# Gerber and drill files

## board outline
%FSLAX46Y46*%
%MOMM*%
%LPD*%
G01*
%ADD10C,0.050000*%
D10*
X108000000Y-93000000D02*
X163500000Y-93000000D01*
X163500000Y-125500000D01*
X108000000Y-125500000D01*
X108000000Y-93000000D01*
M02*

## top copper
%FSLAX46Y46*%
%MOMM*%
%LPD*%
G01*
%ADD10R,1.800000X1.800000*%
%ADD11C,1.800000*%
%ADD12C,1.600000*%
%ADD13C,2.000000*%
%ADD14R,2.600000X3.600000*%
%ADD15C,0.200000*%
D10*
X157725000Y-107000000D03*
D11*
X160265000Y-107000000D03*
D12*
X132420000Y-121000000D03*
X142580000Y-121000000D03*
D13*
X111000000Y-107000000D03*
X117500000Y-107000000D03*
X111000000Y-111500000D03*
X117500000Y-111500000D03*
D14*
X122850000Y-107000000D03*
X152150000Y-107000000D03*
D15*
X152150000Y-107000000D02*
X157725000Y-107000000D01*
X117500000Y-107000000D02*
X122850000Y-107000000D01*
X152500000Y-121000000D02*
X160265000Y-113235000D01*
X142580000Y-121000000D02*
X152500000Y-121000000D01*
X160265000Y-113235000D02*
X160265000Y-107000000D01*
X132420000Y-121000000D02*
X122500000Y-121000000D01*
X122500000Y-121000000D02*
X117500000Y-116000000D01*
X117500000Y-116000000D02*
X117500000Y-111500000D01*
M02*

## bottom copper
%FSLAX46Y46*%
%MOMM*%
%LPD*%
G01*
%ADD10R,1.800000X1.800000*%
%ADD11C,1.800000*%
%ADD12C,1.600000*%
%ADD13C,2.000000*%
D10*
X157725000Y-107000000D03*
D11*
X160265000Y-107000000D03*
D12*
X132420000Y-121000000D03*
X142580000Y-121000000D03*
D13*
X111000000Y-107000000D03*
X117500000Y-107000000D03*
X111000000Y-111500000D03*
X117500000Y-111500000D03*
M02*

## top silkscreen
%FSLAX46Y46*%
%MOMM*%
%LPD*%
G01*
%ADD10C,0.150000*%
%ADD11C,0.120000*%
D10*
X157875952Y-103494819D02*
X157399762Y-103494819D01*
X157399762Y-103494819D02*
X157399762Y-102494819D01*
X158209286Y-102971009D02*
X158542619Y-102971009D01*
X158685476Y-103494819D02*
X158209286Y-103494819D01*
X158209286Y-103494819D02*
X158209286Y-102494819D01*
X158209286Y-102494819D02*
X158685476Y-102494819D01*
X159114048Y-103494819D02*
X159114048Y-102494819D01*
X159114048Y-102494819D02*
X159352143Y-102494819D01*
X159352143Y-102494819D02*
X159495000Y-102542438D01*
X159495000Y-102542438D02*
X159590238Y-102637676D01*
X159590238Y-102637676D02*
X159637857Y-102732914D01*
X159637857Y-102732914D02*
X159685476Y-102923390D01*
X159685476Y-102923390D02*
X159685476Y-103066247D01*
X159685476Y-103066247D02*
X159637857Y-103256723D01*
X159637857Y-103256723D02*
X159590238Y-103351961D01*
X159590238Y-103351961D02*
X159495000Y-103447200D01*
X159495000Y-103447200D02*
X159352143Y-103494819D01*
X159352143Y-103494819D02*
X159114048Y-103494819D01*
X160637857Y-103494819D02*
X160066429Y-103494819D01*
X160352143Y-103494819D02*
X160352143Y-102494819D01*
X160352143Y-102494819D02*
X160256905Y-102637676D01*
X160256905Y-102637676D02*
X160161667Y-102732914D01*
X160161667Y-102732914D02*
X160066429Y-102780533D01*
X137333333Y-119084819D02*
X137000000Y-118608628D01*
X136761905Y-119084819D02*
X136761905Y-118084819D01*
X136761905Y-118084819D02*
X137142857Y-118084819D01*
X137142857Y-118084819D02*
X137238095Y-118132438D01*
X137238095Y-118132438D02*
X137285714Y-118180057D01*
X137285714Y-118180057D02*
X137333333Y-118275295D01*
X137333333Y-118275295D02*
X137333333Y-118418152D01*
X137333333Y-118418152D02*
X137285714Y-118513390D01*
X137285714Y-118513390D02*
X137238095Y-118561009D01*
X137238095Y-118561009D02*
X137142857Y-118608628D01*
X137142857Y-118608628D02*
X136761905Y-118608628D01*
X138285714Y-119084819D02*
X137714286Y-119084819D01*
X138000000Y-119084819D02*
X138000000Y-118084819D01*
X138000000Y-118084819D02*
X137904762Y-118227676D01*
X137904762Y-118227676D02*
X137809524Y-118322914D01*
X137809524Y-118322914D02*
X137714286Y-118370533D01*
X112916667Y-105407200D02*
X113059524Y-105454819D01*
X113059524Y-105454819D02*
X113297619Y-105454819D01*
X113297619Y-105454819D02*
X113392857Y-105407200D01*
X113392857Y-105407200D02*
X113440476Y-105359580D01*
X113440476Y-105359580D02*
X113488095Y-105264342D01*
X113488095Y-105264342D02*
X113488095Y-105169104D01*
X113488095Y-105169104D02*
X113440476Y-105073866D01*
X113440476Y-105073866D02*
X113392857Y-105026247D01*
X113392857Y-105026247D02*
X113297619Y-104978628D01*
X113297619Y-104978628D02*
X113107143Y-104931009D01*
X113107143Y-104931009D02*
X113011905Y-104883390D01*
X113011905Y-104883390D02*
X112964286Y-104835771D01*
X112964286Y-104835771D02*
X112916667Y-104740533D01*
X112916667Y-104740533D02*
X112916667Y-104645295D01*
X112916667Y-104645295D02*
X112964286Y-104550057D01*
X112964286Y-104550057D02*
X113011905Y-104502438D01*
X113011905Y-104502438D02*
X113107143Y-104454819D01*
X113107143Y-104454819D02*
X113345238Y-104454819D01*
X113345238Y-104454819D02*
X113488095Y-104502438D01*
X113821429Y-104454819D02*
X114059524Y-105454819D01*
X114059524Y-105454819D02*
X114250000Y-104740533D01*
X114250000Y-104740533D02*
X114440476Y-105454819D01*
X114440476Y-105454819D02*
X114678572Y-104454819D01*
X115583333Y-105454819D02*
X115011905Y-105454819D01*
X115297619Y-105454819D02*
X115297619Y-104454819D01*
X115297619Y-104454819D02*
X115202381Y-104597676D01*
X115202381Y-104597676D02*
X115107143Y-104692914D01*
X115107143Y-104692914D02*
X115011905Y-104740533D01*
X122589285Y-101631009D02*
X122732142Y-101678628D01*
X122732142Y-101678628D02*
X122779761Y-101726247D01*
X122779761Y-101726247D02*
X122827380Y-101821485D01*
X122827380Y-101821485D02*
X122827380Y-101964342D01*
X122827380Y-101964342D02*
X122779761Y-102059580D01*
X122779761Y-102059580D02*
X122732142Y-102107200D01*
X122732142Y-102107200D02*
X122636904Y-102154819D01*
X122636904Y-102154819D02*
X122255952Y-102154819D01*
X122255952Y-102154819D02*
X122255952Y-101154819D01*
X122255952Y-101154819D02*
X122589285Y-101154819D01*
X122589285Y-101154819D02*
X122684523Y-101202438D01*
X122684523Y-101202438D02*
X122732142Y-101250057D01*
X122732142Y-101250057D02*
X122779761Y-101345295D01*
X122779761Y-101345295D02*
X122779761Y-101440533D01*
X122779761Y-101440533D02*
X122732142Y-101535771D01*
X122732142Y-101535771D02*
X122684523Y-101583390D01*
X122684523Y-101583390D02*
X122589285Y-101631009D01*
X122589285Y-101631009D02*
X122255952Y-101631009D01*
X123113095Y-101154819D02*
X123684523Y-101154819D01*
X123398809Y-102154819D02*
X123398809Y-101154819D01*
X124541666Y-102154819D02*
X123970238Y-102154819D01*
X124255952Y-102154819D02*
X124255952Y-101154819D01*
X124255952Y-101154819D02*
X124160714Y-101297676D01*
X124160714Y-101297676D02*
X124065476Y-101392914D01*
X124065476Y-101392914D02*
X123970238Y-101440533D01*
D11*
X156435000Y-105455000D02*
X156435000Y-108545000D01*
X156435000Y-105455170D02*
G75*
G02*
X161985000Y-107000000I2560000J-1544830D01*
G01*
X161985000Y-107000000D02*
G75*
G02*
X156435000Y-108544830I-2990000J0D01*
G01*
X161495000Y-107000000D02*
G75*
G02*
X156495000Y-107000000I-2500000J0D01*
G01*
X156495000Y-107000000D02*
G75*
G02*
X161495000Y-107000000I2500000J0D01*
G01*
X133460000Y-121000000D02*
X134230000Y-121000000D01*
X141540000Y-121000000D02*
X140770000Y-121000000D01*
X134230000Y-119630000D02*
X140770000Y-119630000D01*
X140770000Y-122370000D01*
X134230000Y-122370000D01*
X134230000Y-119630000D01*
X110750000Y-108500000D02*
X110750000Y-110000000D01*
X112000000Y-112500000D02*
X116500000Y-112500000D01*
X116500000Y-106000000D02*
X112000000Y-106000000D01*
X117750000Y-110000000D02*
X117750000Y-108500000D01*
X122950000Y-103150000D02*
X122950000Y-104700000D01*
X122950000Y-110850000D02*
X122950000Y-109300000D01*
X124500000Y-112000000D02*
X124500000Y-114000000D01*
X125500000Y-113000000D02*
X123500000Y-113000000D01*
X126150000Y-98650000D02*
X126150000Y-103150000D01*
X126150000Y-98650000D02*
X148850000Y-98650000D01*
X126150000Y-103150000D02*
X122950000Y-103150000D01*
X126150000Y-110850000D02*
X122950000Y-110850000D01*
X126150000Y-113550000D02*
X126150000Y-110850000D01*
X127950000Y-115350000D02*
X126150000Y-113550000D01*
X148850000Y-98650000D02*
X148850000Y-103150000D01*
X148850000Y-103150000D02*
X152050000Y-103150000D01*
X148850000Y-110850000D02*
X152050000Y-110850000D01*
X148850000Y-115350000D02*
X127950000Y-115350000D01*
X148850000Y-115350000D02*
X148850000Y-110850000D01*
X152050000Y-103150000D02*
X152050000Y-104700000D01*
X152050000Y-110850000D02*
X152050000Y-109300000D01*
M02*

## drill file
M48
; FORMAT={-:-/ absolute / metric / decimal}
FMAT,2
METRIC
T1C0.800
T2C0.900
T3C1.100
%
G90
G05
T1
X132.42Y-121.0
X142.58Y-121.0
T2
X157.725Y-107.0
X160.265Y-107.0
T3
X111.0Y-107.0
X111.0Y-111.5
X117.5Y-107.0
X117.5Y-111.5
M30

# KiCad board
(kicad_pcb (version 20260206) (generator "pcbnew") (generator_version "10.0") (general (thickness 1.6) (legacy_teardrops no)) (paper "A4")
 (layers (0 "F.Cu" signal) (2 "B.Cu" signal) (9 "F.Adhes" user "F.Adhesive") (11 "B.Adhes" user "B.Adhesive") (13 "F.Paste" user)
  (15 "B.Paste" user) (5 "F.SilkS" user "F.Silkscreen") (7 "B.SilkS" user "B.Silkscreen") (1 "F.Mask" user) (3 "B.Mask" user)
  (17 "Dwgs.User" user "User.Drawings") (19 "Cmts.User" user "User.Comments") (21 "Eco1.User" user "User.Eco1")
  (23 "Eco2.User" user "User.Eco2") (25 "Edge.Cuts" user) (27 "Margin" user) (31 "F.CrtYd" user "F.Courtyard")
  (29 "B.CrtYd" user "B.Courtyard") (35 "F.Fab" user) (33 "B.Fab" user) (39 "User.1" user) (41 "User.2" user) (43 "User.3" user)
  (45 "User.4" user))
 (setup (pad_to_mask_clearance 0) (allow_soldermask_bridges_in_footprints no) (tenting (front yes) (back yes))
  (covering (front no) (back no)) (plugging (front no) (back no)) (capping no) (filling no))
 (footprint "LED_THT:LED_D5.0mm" (layer "F.Cu") (at 157.725 107)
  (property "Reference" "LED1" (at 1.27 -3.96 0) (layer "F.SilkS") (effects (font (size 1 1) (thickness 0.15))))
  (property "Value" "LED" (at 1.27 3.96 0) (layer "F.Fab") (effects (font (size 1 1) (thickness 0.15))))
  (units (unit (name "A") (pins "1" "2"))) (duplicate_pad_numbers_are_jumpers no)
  (fp_line (start -1.29 -1.545) (end -1.29 1.545) (stroke (width 0.12) (type solid)) (layer "F.SilkS"))
  (fp_arc (start -1.29 -1.54483) (mid 2.071779 -2.880495) (end 4.26 0) (stroke (width 0.12) (type solid)) (layer "F.SilkS"))
  (fp_arc (start 4.26 0) (mid 2.071779 2.880495) (end -1.29 1.54483) (stroke (width 0.12) (type solid)) (layer "F.SilkS"))
  (fp_circle (center 1.27 0) (end 3.77 0) (stroke (width 0.12) (type solid)) (fill no) (layer "F.SilkS"))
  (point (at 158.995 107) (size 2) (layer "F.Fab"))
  (pad "1" thru_hole rect (at 0 0) (size 1.8 1.8) (drill 0.9) (layers "*.Cu" "*.Mask") (remove_unused_layers no) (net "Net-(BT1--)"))
  (pad "2" thru_hole circle (at 2.54 0) (size 1.8 1.8) (drill 0.9) (layers "*.Cu" "*.Mask") (remove_unused_layers no) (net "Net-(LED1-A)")))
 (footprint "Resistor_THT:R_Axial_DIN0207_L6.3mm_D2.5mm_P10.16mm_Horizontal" (layer "F.Cu") (at 132.42 121)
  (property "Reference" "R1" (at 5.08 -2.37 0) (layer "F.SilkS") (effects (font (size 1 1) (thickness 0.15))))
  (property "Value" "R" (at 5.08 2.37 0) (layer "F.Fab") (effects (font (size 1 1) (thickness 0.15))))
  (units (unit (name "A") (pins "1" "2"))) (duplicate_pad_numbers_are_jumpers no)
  (fp_line (start 1.04 0) (end 1.81 0) (stroke (width 0.12) (type solid)) (layer "F.SilkS"))
  (fp_line (start 9.12 0) (end 8.35 0) (stroke (width 0.12) (type solid)) (layer "F.SilkS"))
  (fp_rect (start 1.81 -1.37) (end 8.35 1.37) (stroke (width 0.12) (type solid)) (fill no) (layer "F.SilkS"))
  (pad "1" thru_hole circle (at 0 0) (size 1.6 1.6) (drill 0.8) (layers "*.Cu" "*.Mask") (remove_unused_layers no) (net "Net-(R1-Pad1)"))
  (pad "2" thru_hole circle (at 10.16 0) (size 1.6 1.6) (drill 0.8) (layers "*.Cu" "*.Mask") (remove_unused_layers no) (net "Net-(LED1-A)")))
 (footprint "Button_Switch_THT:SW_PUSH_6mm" (layer "F.Cu") (at 111 107)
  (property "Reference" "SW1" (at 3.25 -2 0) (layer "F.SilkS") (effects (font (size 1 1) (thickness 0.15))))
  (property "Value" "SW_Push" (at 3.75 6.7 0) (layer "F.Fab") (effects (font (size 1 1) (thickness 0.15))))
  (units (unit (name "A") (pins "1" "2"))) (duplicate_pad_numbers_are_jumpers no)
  (fp_line (start -0.25 1.5) (end -0.25 3) (stroke (width 0.12) (type solid)) (layer "F.SilkS"))
  (fp_line (start 1 5.5) (end 5.5 5.5) (stroke (width 0.12) (type solid)) (layer "F.SilkS"))
  (fp_line (start 5.5 -1) (end 1 -1) (stroke (width 0.12) (type solid)) (layer "F.SilkS"))
  (fp_line (start 6.75 3) (end 6.75 1.5) (stroke (width 0.12) (type solid)) (layer "F.SilkS"))
  (pad "1" thru_hole circle (at 0 0 90) (size 2 2) (drill 1.1) (layers "*.Cu" "*.Mask") (remove_unused_layers no) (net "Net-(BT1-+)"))
  (pad "1" thru_hole circle (at 6.5 0 90) (size 2 2) (drill 1.1) (layers "*.Cu" "*.Mask") (remove_unused_layers no) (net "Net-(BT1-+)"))
  (pad "2" thru_hole circle (at 0 4.5 90) (size 2 2) (drill 1.1) (layers "*.Cu" "*.Mask") (remove_unused_layers no) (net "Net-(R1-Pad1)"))
  (pad "2" thru_hole circle (at 6.5 4.5 90) (size 2 2) (drill 1.1) (layers "*.Cu" "*.Mask") (remove_unused_layers no) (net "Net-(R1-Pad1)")))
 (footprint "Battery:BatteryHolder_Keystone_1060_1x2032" (layer "F.Cu") (at 137.5 107)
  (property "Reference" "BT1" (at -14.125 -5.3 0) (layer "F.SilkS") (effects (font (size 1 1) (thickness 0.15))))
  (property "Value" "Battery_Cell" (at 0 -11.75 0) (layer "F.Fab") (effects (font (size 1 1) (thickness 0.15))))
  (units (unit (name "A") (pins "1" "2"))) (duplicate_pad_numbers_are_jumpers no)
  (fp_line (start -14.55 -3.85) (end -14.55 -2.3) (stroke (width 0.12) (type solid)) (layer "F.SilkS"))
  (fp_line (start -14.55 3.85) (end -14.55 2.3) (stroke (width 0.12) (type solid)) (layer "F.SilkS"))
  (fp_line (start -13 5) (end -13 7) (stroke (width 0.12) (type solid)) (layer "F.SilkS"))
  (fp_line (start -12 6) (end -14 6) (stroke (width 0.12) (type solid)) (layer "F.SilkS"))
  (fp_line (start -11.35 -8.35) (end -11.35 -3.85) (stroke (width 0.12) (type solid)) (layer "F.SilkS"))
  (fp_line (start -11.35 -8.35) (end 11.35 -8.35) (stroke (width 0.12) (type solid)) (layer "F.SilkS"))
  (fp_line (start -11.35 -3.85) (end -14.55 -3.85) (stroke (width 0.12) (type solid)) (layer "F.SilkS"))
  (fp_line (start -11.35 3.85) (end -14.55 3.85) (stroke (width 0.12) (type solid)) (layer "F.SilkS"))
  (fp_line (start -11.35 6.55) (end -11.35 3.85) (stroke (width 0.12) (type solid)) (layer "F.SilkS"))
  (fp_line (start -9.55 8.35) (end -11.35 6.55) (stroke (width 0.12) (type solid)) (layer "F.SilkS"))
  (fp_line (start 11.35 -8.35) (end 11.35 -3.85) (stroke (width 0.12) (type solid)) (layer "F.SilkS"))
  (fp_line (start 11.35 -3.85) (end 14.55 -3.85) (stroke (width 0.12) (type solid)) (layer "F.SilkS"))
  (fp_line (start 11.35 3.85) (end 14.55 3.85) (stroke (width 0.12) (type solid)) (layer "F.SilkS"))
  (fp_line (start 11.35 8.35) (end -9.55 8.35) (stroke (width 0.12) (type solid)) (layer "F.SilkS"))
  (fp_line (start 11.35 8.35) (end 11.35 3.85) (stroke (width 0.12) (type solid)) (layer "F.SilkS"))
  (fp_line (start 14.55 -3.85) (end 14.55 -2.3) (stroke (width 0.12) (type solid)) (layer "F.SilkS"))
  (fp_line (start 14.55 3.85) (end 14.55 2.3) (stroke (width 0.12) (type solid)) (layer "F.SilkS"))
  (pad "1" smd rect (at -14.65 0 180) (size 2.6 3.6) (layers "F.Cu" "F.Mask" "F.Paste") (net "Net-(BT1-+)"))
  (pad "2" smd rect (at 14.65 0 180) (size 2.6 3.6) (layers "F.Cu" "F.Mask" "F.Paste") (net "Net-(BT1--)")))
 (gr_rect (start 108 93) (end 163.5 125.5) (stroke (width 0.05) (type default)) (fill no) (layer "Edge.Cuts"))
 (segment (start 152.15 107) (end 157.725 107) (width 0.2) (layer "F.Cu") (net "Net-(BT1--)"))
 (segment (start 117.5 107) (end 122.85 107) (width 0.2) (layer "F.Cu") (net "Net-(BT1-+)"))
 (segment (start 152.5 121) (end 160.265 113.235) (width 0.2) (layer "F.Cu") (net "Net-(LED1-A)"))
 (segment (start 142.58 121) (end 152.5 121) (width 0.2) (layer "F.Cu") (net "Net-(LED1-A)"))
 (segment (start 160.265 113.235) (end 160.265 107) (width 0.2) (layer "F.Cu") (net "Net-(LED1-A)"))
 (segment (start 132.42 121) (end 122.5 121) (width 0.2) (layer "F.Cu") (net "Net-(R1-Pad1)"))
 (segment (start 122.5 121) (end 117.5 116) (width 0.2) (layer "F.Cu") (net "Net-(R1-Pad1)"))
 (segment (start 117.5 116) (end 117.5 111.5) (width 0.2) (layer "F.Cu") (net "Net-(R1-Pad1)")))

